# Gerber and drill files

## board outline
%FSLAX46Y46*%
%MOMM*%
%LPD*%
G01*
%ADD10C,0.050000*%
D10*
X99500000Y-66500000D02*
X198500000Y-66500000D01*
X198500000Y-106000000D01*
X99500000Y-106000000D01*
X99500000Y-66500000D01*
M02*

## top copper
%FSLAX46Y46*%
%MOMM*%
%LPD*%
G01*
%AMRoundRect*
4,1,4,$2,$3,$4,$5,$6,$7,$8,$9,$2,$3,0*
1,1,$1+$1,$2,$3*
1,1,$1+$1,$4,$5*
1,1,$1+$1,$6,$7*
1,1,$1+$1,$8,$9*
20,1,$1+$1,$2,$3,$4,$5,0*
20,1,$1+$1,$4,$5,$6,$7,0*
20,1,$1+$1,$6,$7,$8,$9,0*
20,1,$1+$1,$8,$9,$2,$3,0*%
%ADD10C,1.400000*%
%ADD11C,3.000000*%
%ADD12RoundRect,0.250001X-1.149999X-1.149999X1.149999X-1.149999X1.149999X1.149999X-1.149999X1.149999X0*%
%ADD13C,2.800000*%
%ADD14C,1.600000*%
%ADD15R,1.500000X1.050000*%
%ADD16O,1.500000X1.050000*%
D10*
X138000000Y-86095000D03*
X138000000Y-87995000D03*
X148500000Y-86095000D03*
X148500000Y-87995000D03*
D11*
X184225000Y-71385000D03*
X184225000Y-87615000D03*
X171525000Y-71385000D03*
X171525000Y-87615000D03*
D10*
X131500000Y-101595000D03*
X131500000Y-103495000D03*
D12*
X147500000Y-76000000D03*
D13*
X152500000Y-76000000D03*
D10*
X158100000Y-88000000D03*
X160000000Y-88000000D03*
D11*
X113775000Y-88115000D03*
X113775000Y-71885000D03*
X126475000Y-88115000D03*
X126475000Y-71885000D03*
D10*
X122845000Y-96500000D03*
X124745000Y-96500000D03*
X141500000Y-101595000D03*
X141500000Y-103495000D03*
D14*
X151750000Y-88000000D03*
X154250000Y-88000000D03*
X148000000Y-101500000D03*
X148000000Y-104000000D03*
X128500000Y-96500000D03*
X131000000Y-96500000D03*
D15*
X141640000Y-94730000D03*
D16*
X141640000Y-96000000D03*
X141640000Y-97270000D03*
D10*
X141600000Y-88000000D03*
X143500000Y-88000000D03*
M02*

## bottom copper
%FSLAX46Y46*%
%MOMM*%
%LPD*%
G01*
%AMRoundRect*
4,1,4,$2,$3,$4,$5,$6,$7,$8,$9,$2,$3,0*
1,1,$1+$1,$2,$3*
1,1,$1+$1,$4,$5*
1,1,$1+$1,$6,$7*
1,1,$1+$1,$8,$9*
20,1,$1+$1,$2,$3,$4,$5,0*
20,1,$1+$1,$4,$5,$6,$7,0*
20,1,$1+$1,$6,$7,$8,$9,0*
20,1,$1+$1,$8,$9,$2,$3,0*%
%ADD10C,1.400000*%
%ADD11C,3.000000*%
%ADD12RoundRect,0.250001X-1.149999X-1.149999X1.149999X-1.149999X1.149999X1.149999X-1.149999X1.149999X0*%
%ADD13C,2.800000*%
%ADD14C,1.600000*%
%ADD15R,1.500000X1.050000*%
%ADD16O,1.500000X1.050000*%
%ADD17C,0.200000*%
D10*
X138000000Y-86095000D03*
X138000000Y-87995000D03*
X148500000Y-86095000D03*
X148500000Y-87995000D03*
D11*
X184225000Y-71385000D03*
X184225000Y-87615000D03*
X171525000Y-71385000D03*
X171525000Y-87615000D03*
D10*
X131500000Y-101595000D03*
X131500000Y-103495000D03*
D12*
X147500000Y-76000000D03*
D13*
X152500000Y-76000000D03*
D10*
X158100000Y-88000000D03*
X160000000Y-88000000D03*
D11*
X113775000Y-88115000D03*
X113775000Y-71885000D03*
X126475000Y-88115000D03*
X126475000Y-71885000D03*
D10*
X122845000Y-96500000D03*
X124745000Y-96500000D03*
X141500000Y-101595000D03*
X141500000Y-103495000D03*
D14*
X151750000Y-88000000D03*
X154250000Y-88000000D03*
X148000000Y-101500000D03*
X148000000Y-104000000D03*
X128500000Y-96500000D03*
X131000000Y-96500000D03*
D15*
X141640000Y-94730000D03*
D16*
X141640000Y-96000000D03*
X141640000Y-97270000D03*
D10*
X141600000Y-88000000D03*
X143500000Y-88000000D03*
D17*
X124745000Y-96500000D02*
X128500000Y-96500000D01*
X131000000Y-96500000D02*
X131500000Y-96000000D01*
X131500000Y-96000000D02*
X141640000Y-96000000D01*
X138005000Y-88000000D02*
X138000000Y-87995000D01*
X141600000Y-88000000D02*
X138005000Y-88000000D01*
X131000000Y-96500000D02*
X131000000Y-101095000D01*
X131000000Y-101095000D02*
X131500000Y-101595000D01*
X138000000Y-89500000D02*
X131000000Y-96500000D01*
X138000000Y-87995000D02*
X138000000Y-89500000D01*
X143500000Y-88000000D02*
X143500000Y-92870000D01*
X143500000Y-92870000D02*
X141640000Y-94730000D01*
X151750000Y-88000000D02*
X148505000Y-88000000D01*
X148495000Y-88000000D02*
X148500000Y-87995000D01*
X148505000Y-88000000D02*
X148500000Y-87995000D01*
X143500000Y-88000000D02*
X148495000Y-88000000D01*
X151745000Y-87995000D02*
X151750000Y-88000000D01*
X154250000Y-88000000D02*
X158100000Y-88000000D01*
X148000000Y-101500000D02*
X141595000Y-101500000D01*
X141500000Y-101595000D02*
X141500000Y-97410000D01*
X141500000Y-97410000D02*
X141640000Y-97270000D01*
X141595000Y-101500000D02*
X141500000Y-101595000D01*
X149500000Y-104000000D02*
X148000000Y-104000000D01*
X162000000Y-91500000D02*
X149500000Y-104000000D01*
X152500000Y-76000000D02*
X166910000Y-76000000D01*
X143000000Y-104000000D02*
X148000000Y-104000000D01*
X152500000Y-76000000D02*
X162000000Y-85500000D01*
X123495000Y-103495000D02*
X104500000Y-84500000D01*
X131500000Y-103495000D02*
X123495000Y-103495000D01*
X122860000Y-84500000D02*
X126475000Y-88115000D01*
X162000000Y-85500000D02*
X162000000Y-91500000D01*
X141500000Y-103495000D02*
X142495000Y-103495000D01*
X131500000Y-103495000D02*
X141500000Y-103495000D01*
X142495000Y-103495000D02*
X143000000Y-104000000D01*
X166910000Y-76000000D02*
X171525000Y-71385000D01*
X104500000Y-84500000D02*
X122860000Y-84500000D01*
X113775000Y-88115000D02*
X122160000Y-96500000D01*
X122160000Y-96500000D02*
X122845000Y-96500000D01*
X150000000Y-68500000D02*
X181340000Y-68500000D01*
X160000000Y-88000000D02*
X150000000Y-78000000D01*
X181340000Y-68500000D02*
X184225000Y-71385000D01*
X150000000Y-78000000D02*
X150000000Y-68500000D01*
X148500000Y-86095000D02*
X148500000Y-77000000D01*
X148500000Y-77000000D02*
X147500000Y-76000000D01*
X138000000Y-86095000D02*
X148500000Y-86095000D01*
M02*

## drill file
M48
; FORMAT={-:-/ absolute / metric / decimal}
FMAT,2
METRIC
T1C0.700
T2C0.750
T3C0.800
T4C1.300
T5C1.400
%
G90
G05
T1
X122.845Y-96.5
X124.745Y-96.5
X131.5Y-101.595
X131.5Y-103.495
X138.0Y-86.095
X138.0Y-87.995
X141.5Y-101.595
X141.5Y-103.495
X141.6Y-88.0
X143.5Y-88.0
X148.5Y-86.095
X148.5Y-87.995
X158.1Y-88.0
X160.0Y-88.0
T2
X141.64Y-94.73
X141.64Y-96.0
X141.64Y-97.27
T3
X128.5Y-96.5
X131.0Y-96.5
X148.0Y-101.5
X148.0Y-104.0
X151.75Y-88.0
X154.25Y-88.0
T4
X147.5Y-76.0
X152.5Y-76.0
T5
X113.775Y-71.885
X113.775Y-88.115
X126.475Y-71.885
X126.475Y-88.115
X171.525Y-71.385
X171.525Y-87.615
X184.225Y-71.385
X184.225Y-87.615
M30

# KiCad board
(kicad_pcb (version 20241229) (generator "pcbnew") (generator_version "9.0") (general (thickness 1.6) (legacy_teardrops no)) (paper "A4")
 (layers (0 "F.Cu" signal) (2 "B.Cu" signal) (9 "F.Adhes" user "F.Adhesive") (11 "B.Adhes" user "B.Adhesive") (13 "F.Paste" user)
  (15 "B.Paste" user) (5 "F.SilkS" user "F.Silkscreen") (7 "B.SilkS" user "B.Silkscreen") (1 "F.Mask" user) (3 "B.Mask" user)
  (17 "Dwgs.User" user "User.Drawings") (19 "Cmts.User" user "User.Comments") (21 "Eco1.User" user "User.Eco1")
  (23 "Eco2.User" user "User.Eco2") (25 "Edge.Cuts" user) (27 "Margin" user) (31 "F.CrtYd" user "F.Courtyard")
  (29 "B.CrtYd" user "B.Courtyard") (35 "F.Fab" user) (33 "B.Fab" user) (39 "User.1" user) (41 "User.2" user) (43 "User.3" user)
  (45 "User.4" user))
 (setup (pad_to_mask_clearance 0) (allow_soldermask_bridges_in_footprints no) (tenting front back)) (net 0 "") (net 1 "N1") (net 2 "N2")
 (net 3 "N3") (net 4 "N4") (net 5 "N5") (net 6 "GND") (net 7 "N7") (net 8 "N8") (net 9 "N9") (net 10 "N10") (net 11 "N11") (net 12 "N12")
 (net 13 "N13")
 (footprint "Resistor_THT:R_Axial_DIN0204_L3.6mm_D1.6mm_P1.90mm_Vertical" (layer "F.Cu") (at 138 86.095 -90)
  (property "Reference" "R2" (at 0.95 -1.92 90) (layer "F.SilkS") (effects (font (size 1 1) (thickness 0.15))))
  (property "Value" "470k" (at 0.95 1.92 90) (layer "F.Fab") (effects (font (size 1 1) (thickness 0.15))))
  (pad "1" thru_hole circle (at 0 0 270) (size 1.4 1.4) (drill 0.7) (layers "*.Cu" "*.Mask") (remove_unused_layers no) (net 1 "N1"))
  (pad "2" thru_hole circle (at 1.9 0 270) (size 1.4 1.4) (drill 0.7) (layers "*.Cu" "*.Mask") (remove_unused_layers no) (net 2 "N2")))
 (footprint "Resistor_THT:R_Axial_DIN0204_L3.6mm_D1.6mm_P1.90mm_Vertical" (layer "F.Cu") (at 148.5 86.095 -90)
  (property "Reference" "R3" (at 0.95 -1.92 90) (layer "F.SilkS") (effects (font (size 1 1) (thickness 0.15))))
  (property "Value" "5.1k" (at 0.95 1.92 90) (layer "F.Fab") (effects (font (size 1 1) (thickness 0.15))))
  (pad "1" thru_hole circle (at 0 0 270) (size 1.4 1.4) (drill 0.7) (layers "*.Cu" "*.Mask") (remove_unused_layers no) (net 1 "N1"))
  (pad "2" thru_hole circle (at 1.9 0 270) (size 1.4 1.4) (drill 0.7) (layers "*.Cu" "*.Mask") (remove_unused_layers no) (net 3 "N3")))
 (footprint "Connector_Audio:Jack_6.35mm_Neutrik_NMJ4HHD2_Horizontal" (layer "F.Cu") (at 171.525 71.385)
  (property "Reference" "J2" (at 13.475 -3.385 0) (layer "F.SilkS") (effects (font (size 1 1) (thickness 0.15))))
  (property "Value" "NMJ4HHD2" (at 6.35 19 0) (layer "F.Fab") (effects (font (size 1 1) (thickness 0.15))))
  (pad "S" thru_hole circle (at 12.7 0) (size 3 3) (drill 1.4) (layers "*.Cu" "*.Mask") (remove_unused_layers no) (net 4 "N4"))
  (pad "SN" thru_hole circle (at 12.7 16.23) (size 3 3) (drill 1.4) (layers "*.Cu" "*.Mask") (remove_unused_layers no) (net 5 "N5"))
  (pad "T" thru_hole circle (at 0 0) (size 3 3) (drill 1.4) (layers "*.Cu" "*.Mask") (remove_unused_layers no) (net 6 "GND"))
  (pad "TN" thru_hole circle (at 0 16.23) (size 3 3) (drill 1.4) (layers "*.Cu" "*.Mask") (remove_unused_layers no) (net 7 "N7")))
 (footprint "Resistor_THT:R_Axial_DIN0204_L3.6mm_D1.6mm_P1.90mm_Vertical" (layer "F.Cu") (at 131.5 101.595 -90)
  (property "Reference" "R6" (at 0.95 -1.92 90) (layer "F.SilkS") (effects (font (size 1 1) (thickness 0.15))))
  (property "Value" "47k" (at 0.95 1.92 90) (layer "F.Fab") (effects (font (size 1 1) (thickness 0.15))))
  (pad "1" thru_hole circle (at 0 0 270) (size 1.4 1.4) (drill 0.7) (layers "*.Cu" "*.Mask") (remove_unused_layers no) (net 2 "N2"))
  (pad "2" thru_hole circle (at 1.9 0 270) (size 1.4 1.4) (drill 0.7) (layers "*.Cu" "*.Mask") (remove_unused_layers no) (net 6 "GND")))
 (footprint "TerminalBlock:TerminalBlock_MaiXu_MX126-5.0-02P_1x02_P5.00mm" (layer "F.Cu") (at 147.5 76)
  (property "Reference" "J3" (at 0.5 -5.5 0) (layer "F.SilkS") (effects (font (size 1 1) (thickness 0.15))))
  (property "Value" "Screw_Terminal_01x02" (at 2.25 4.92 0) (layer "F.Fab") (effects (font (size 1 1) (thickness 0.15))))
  (pad "1" thru_hole roundrect (at 0 0) (size 2.8 2.8) (drill 1.3) (layers "*.Cu" "*.Mask") (remove_unused_layers no)
   (roundrect_rratio 0.089286) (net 1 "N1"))
  (pad "2" thru_hole circle (at 5 0) (size 2.8 2.8) (drill 1.3) (layers "*.Cu" "*.Mask") (remove_unused_layers no) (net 6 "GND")))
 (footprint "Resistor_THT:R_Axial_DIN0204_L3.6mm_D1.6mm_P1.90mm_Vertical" (layer "F.Cu") (at 158.1 88)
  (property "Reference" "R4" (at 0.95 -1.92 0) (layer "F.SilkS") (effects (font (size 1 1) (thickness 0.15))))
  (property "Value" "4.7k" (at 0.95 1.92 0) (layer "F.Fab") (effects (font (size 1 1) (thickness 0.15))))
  (pad "1" thru_hole circle (at 0 0) (size 1.4 1.4) (drill 0.7) (layers "*.Cu" "*.Mask") (remove_unused_layers no) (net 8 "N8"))
  (pad "2" thru_hole circle (at 1.9 0) (size 1.4 1.4) (drill 0.7) (layers "*.Cu" "*.Mask") (remove_unused_layers no) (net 4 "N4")))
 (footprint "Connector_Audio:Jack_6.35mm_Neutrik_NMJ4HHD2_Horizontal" (layer "F.Cu") (at 126.475 88.115 180)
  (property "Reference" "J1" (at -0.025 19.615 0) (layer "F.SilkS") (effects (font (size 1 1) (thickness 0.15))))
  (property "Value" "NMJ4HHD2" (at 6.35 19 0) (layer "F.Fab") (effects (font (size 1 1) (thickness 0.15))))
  (pad "S" thru_hole circle (at 12.7 0 180) (size 3 3) (drill 1.4) (layers "*.Cu" "*.Mask") (remove_unused_layers no) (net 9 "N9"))
  (pad "SN" thru_hole circle (at 12.7 16.23 180) (size 3 3) (drill 1.4) (layers "*.Cu" "*.Mask") (remove_unused_layers no) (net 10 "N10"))
  (pad "T" thru_hole circle (at 0 0 180) (size 3 3) (drill 1.4) (layers "*.Cu" "*.Mask") (remove_unused_layers no) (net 6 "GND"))
  (pad "TN" thru_hole circle (at 0 16.23 180) (size 3 3) (drill 1.4) (layers "*.Cu" "*.Mask") (remove_unused_layers no) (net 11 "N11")))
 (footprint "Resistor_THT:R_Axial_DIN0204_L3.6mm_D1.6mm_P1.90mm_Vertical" (layer "F.Cu") (at 122.845 96.5)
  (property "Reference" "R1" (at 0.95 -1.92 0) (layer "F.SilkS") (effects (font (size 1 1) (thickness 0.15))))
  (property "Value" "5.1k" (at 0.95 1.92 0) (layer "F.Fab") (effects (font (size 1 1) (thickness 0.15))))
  (pad "1" thru_hole circle (at 0 0) (size 1.4 1.4) (drill 0.7) (layers "*.Cu" "*.Mask") (remove_unused_layers no) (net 9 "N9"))
  (pad "2" thru_hole circle (at 1.9 0) (size 1.4 1.4) (drill 0.7) (layers "*.Cu" "*.Mask") (remove_unused_layers no) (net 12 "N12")))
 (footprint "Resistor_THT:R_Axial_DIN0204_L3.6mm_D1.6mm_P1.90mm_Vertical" (layer "F.Cu") (at 141.5 101.595 -90)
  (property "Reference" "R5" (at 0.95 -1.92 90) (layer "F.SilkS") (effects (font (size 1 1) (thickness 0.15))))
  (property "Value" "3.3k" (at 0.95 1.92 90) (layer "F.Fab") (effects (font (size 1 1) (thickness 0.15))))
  (pad "1" thru_hole circle (at 0 0 270) (size 1.4 1.4) (drill 0.7) (layers "*.Cu" "*.Mask") (remove_unused_layers no) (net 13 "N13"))
  (pad "2" thru_hole circle (at 1.9 0 270) (size 1.4 1.4) (drill 0.7) (layers "*.Cu" "*.Mask") (remove_unused_layers no) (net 6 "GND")))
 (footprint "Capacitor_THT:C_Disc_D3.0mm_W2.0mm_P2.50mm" (layer "F.Cu") (at 151.75 88)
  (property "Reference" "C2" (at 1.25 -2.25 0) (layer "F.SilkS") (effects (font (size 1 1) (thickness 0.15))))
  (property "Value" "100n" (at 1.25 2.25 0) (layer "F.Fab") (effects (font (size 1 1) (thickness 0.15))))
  (pad "1" thru_hole circle (at 0 0) (size 1.6 1.6) (drill 0.8) (layers "*.Cu" "*.Mask") (remove_unused_layers no) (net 3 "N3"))
  (pad "2" thru_hole circle (at 2.5 0) (size 1.6 1.6) (drill 0.8) (layers "*.Cu" "*.Mask") (remove_unused_layers no) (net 8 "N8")))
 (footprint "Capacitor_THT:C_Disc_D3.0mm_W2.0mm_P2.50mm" (layer "F.Cu") (at 148 101.5 -90)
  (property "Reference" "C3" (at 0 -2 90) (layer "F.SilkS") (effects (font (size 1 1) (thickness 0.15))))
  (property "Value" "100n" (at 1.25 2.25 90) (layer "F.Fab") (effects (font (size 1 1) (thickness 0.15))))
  (pad "1" thru_hole circle (at 0 0 270) (size 1.6 1.6) (drill 0.8) (layers "*.Cu" "*.Mask") (remove_unused_layers no) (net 13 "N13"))
  (pad "2" thru_hole circle (at 2.5 0 270) (size 1.6 1.6) (drill 0.8) (layers "*.Cu" "*.Mask") (remove_unused_layers no) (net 6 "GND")))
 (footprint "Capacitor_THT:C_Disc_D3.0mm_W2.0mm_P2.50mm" (layer "F.Cu") (at 128.5 96.5)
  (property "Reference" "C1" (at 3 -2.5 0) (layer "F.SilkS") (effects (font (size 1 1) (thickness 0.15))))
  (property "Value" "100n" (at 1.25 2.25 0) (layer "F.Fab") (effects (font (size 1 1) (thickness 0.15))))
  (pad "1" thru_hole circle (at 0 0) (size 1.6 1.6) (drill 0.8) (layers "*.Cu" "*.Mask") (remove_unused_layers no) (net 12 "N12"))
  (pad "2" thru_hole circle (at 2.5 0) (size 1.6 1.6) (drill 0.8) (layers "*.Cu" "*.Mask") (remove_unused_layers no) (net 2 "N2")))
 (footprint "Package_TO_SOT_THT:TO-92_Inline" (layer "F.Cu") (at 141.64 94.73 -90)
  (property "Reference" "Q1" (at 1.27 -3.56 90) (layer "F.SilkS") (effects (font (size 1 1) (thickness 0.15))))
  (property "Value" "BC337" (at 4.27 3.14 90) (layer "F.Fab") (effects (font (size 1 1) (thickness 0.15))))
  (pad "1" thru_hole rect (at 0 0 270) (size 1.05 1.5) (drill 0.75) (layers "*.Cu" "*.Mask") (remove_unused_layers no) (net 3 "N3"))
  (pad "2" thru_hole oval (at 1.27 0 270) (size 1.05 1.5) (drill 0.75) (layers "*.Cu" "*.Mask") (remove_unused_layers no) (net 2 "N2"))
  (pad "3" thru_hole oval (at 2.54 0 270) (size 1.05 1.5) (drill 0.75) (layers "*.Cu" "*.Mask") (remove_unused_layers no) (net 13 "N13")))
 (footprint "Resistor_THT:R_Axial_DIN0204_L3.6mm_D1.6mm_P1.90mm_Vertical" (layer "F.Cu") (at 141.6 88)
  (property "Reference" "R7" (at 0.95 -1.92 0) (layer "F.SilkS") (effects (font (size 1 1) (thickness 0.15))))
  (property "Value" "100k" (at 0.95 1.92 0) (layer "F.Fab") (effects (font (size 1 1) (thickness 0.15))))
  (pad "1" thru_hole circle (at 0 0) (size 1.4 1.4) (drill 0.7) (layers "*.Cu" "*.Mask") (remove_unused_layers no) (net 2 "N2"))
  (pad "2" thru_hole circle (at 1.9 0) (size 1.4 1.4) (drill 0.7) (layers "*.Cu" "*.Mask") (remove_unused_layers no) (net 3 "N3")))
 (gr_rect (start 99.5 66.5) (end 198.5 106) (stroke (width 0.05) (type default)) (fill no) (layer "Edge.Cuts"))
 (segment (start 124.745 96.5) (end 128.5 96.5) (width 0.2) (layer "B.Cu") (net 12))
 (segment (start 131 96.5) (end 131.5 96) (width 0.2) (layer "B.Cu") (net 2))
 (segment (start 131.5 96) (end 141.64 96) (width 0.2) (layer "B.Cu") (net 2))
 (segment (start 138.005 88) (end 138 87.995) (width 0.2) (layer "B.Cu") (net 2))
 (segment (start 141.6 88) (end 138.005 88) (width 0.2) (layer "B.Cu") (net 2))
 (segment (start 131 96.5) (end 131 101.095) (width 0.2) (layer "B.Cu") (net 2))
 (segment (start 131 101.095) (end 131.5 101.595) (width 0.2) (layer "B.Cu") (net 2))
 (segment (start 138 89.5) (end 131 96.5) (width 0.2) (layer "B.Cu") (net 2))
 (segment (start 138 87.995) (end 138 89.5) (width 0.2) (layer "B.Cu") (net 2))
 (segment (start 143.5 88) (end 143.5 92.87) (width 0.2) (layer "B.Cu") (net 3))
 (segment (start 143.5 92.87) (end 141.64 94.73) (width 0.2) (layer "B.Cu") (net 3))
 (segment (start 151.75 88) (end 148.505 88) (width 0.2) (layer "B.Cu") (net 3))
 (segment (start 148.495 88) (end 148.5 87.995) (width 0.2) (layer "B.Cu") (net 3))
 (segment (start 148.505 88) (end 148.5 87.995) (width 0.2) (layer "B.Cu") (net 3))
 (segment (start 143.5 88) (end 148.495 88) (width 0.2) (layer "B.Cu") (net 3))
 (segment (start 151.745 87.995) (end 151.75 88) (width 0.2) (layer "B.Cu") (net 3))
 (segment (start 154.25 88) (end 158.1 88) (width 0.2) (layer "B.Cu") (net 8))
 (segment (start 148 101.5) (end 141.595 101.5) (width 0.2) (layer "B.Cu") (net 13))
 (segment (start 141.5 101.595) (end 141.5 97.41) (width 0.2) (layer "B.Cu") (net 13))
 (segment (start 141.5 97.41) (end 141.64 97.27) (width 0.2) (layer "B.Cu") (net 13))
 (segment (start 141.595 101.5) (end 141.5 101.595) (width 0.2) (layer "B.Cu") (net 13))
 (segment (start 149.5 104) (end 148 104) (width 0.2) (layer "B.Cu") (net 6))
 (segment (start 162 91.5) (end 149.5 104) (width 0.2) (layer "B.Cu") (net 6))
 (segment (start 152.5 76) (end 166.91 76) (width 0.2) (layer "B.Cu") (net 6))
 (segment (start 143 104) (end 148 104) (width 0.2) (layer "B.Cu") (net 6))
 (segment (start 152.5 76) (end 162 85.5) (width 0.2) (layer "B.Cu") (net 6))
 (segment (start 123.495 103.495) (end 104.5 84.5) (width 0.2) (layer "B.Cu") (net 6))
 (segment (start 131.5 103.495) (end 123.495 103.495) (width 0.2) (layer "B.Cu") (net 6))
 (segment (start 122.86 84.5) (end 126.475 88.115) (width 0.2) (layer "B.Cu") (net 6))
 (segment (start 162 85.5) (end 162 91.5) (width 0.2) (layer "B.Cu") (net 6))
 (segment (start 141.5 103.495) (end 142.495 103.495) (width 0.2) (layer "B.Cu") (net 6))
 (segment (start 131.5 103.495) (end 141.5 103.495) (width 0.2) (layer "B.Cu") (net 6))
 (segment (start 142.495 103.495) (end 143 104) (width 0.2) (layer "B.Cu") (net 6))
 (segment (start 166.91 76) (end 171.525 71.385) (width 0.2) (layer "B.Cu") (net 6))
 (segment (start 104.5 84.5) (end 122.86 84.5) (width 0.2) (layer "B.Cu") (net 6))
 (segment (start 113.775 88.115) (end 122.16 96.5) (width 0.2) (layer "B.Cu") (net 9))
 (segment (start 122.16 96.5) (end 122.845 96.5) (width 0.2) (layer "B.Cu") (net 9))
 (segment (start 150 68.5) (end 181.34 68.5) (width 0.2) (layer "B.Cu") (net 4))
 (segment (start 160 88) (end 150 78) (width 0.2) (layer "B.Cu") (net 4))
 (segment (start 181.34 68.5) (end 184.225 71.385) (width 0.2) (layer "B.Cu") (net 4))
 (segment (start 150 78) (end 150 68.5) (width 0.2) (layer "B.Cu") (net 4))
 (segment (start 148.5 86.095) (end 148.5 77) (width 0.2) (layer "B.Cu") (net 1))
 (segment (start 148.5 77) (end 147.5 76) (width 0.2) (layer "B.Cu") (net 1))
 (segment (start 138 86.095) (end 148.5 86.095) (width 0.2) (layer "B.Cu") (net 1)))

